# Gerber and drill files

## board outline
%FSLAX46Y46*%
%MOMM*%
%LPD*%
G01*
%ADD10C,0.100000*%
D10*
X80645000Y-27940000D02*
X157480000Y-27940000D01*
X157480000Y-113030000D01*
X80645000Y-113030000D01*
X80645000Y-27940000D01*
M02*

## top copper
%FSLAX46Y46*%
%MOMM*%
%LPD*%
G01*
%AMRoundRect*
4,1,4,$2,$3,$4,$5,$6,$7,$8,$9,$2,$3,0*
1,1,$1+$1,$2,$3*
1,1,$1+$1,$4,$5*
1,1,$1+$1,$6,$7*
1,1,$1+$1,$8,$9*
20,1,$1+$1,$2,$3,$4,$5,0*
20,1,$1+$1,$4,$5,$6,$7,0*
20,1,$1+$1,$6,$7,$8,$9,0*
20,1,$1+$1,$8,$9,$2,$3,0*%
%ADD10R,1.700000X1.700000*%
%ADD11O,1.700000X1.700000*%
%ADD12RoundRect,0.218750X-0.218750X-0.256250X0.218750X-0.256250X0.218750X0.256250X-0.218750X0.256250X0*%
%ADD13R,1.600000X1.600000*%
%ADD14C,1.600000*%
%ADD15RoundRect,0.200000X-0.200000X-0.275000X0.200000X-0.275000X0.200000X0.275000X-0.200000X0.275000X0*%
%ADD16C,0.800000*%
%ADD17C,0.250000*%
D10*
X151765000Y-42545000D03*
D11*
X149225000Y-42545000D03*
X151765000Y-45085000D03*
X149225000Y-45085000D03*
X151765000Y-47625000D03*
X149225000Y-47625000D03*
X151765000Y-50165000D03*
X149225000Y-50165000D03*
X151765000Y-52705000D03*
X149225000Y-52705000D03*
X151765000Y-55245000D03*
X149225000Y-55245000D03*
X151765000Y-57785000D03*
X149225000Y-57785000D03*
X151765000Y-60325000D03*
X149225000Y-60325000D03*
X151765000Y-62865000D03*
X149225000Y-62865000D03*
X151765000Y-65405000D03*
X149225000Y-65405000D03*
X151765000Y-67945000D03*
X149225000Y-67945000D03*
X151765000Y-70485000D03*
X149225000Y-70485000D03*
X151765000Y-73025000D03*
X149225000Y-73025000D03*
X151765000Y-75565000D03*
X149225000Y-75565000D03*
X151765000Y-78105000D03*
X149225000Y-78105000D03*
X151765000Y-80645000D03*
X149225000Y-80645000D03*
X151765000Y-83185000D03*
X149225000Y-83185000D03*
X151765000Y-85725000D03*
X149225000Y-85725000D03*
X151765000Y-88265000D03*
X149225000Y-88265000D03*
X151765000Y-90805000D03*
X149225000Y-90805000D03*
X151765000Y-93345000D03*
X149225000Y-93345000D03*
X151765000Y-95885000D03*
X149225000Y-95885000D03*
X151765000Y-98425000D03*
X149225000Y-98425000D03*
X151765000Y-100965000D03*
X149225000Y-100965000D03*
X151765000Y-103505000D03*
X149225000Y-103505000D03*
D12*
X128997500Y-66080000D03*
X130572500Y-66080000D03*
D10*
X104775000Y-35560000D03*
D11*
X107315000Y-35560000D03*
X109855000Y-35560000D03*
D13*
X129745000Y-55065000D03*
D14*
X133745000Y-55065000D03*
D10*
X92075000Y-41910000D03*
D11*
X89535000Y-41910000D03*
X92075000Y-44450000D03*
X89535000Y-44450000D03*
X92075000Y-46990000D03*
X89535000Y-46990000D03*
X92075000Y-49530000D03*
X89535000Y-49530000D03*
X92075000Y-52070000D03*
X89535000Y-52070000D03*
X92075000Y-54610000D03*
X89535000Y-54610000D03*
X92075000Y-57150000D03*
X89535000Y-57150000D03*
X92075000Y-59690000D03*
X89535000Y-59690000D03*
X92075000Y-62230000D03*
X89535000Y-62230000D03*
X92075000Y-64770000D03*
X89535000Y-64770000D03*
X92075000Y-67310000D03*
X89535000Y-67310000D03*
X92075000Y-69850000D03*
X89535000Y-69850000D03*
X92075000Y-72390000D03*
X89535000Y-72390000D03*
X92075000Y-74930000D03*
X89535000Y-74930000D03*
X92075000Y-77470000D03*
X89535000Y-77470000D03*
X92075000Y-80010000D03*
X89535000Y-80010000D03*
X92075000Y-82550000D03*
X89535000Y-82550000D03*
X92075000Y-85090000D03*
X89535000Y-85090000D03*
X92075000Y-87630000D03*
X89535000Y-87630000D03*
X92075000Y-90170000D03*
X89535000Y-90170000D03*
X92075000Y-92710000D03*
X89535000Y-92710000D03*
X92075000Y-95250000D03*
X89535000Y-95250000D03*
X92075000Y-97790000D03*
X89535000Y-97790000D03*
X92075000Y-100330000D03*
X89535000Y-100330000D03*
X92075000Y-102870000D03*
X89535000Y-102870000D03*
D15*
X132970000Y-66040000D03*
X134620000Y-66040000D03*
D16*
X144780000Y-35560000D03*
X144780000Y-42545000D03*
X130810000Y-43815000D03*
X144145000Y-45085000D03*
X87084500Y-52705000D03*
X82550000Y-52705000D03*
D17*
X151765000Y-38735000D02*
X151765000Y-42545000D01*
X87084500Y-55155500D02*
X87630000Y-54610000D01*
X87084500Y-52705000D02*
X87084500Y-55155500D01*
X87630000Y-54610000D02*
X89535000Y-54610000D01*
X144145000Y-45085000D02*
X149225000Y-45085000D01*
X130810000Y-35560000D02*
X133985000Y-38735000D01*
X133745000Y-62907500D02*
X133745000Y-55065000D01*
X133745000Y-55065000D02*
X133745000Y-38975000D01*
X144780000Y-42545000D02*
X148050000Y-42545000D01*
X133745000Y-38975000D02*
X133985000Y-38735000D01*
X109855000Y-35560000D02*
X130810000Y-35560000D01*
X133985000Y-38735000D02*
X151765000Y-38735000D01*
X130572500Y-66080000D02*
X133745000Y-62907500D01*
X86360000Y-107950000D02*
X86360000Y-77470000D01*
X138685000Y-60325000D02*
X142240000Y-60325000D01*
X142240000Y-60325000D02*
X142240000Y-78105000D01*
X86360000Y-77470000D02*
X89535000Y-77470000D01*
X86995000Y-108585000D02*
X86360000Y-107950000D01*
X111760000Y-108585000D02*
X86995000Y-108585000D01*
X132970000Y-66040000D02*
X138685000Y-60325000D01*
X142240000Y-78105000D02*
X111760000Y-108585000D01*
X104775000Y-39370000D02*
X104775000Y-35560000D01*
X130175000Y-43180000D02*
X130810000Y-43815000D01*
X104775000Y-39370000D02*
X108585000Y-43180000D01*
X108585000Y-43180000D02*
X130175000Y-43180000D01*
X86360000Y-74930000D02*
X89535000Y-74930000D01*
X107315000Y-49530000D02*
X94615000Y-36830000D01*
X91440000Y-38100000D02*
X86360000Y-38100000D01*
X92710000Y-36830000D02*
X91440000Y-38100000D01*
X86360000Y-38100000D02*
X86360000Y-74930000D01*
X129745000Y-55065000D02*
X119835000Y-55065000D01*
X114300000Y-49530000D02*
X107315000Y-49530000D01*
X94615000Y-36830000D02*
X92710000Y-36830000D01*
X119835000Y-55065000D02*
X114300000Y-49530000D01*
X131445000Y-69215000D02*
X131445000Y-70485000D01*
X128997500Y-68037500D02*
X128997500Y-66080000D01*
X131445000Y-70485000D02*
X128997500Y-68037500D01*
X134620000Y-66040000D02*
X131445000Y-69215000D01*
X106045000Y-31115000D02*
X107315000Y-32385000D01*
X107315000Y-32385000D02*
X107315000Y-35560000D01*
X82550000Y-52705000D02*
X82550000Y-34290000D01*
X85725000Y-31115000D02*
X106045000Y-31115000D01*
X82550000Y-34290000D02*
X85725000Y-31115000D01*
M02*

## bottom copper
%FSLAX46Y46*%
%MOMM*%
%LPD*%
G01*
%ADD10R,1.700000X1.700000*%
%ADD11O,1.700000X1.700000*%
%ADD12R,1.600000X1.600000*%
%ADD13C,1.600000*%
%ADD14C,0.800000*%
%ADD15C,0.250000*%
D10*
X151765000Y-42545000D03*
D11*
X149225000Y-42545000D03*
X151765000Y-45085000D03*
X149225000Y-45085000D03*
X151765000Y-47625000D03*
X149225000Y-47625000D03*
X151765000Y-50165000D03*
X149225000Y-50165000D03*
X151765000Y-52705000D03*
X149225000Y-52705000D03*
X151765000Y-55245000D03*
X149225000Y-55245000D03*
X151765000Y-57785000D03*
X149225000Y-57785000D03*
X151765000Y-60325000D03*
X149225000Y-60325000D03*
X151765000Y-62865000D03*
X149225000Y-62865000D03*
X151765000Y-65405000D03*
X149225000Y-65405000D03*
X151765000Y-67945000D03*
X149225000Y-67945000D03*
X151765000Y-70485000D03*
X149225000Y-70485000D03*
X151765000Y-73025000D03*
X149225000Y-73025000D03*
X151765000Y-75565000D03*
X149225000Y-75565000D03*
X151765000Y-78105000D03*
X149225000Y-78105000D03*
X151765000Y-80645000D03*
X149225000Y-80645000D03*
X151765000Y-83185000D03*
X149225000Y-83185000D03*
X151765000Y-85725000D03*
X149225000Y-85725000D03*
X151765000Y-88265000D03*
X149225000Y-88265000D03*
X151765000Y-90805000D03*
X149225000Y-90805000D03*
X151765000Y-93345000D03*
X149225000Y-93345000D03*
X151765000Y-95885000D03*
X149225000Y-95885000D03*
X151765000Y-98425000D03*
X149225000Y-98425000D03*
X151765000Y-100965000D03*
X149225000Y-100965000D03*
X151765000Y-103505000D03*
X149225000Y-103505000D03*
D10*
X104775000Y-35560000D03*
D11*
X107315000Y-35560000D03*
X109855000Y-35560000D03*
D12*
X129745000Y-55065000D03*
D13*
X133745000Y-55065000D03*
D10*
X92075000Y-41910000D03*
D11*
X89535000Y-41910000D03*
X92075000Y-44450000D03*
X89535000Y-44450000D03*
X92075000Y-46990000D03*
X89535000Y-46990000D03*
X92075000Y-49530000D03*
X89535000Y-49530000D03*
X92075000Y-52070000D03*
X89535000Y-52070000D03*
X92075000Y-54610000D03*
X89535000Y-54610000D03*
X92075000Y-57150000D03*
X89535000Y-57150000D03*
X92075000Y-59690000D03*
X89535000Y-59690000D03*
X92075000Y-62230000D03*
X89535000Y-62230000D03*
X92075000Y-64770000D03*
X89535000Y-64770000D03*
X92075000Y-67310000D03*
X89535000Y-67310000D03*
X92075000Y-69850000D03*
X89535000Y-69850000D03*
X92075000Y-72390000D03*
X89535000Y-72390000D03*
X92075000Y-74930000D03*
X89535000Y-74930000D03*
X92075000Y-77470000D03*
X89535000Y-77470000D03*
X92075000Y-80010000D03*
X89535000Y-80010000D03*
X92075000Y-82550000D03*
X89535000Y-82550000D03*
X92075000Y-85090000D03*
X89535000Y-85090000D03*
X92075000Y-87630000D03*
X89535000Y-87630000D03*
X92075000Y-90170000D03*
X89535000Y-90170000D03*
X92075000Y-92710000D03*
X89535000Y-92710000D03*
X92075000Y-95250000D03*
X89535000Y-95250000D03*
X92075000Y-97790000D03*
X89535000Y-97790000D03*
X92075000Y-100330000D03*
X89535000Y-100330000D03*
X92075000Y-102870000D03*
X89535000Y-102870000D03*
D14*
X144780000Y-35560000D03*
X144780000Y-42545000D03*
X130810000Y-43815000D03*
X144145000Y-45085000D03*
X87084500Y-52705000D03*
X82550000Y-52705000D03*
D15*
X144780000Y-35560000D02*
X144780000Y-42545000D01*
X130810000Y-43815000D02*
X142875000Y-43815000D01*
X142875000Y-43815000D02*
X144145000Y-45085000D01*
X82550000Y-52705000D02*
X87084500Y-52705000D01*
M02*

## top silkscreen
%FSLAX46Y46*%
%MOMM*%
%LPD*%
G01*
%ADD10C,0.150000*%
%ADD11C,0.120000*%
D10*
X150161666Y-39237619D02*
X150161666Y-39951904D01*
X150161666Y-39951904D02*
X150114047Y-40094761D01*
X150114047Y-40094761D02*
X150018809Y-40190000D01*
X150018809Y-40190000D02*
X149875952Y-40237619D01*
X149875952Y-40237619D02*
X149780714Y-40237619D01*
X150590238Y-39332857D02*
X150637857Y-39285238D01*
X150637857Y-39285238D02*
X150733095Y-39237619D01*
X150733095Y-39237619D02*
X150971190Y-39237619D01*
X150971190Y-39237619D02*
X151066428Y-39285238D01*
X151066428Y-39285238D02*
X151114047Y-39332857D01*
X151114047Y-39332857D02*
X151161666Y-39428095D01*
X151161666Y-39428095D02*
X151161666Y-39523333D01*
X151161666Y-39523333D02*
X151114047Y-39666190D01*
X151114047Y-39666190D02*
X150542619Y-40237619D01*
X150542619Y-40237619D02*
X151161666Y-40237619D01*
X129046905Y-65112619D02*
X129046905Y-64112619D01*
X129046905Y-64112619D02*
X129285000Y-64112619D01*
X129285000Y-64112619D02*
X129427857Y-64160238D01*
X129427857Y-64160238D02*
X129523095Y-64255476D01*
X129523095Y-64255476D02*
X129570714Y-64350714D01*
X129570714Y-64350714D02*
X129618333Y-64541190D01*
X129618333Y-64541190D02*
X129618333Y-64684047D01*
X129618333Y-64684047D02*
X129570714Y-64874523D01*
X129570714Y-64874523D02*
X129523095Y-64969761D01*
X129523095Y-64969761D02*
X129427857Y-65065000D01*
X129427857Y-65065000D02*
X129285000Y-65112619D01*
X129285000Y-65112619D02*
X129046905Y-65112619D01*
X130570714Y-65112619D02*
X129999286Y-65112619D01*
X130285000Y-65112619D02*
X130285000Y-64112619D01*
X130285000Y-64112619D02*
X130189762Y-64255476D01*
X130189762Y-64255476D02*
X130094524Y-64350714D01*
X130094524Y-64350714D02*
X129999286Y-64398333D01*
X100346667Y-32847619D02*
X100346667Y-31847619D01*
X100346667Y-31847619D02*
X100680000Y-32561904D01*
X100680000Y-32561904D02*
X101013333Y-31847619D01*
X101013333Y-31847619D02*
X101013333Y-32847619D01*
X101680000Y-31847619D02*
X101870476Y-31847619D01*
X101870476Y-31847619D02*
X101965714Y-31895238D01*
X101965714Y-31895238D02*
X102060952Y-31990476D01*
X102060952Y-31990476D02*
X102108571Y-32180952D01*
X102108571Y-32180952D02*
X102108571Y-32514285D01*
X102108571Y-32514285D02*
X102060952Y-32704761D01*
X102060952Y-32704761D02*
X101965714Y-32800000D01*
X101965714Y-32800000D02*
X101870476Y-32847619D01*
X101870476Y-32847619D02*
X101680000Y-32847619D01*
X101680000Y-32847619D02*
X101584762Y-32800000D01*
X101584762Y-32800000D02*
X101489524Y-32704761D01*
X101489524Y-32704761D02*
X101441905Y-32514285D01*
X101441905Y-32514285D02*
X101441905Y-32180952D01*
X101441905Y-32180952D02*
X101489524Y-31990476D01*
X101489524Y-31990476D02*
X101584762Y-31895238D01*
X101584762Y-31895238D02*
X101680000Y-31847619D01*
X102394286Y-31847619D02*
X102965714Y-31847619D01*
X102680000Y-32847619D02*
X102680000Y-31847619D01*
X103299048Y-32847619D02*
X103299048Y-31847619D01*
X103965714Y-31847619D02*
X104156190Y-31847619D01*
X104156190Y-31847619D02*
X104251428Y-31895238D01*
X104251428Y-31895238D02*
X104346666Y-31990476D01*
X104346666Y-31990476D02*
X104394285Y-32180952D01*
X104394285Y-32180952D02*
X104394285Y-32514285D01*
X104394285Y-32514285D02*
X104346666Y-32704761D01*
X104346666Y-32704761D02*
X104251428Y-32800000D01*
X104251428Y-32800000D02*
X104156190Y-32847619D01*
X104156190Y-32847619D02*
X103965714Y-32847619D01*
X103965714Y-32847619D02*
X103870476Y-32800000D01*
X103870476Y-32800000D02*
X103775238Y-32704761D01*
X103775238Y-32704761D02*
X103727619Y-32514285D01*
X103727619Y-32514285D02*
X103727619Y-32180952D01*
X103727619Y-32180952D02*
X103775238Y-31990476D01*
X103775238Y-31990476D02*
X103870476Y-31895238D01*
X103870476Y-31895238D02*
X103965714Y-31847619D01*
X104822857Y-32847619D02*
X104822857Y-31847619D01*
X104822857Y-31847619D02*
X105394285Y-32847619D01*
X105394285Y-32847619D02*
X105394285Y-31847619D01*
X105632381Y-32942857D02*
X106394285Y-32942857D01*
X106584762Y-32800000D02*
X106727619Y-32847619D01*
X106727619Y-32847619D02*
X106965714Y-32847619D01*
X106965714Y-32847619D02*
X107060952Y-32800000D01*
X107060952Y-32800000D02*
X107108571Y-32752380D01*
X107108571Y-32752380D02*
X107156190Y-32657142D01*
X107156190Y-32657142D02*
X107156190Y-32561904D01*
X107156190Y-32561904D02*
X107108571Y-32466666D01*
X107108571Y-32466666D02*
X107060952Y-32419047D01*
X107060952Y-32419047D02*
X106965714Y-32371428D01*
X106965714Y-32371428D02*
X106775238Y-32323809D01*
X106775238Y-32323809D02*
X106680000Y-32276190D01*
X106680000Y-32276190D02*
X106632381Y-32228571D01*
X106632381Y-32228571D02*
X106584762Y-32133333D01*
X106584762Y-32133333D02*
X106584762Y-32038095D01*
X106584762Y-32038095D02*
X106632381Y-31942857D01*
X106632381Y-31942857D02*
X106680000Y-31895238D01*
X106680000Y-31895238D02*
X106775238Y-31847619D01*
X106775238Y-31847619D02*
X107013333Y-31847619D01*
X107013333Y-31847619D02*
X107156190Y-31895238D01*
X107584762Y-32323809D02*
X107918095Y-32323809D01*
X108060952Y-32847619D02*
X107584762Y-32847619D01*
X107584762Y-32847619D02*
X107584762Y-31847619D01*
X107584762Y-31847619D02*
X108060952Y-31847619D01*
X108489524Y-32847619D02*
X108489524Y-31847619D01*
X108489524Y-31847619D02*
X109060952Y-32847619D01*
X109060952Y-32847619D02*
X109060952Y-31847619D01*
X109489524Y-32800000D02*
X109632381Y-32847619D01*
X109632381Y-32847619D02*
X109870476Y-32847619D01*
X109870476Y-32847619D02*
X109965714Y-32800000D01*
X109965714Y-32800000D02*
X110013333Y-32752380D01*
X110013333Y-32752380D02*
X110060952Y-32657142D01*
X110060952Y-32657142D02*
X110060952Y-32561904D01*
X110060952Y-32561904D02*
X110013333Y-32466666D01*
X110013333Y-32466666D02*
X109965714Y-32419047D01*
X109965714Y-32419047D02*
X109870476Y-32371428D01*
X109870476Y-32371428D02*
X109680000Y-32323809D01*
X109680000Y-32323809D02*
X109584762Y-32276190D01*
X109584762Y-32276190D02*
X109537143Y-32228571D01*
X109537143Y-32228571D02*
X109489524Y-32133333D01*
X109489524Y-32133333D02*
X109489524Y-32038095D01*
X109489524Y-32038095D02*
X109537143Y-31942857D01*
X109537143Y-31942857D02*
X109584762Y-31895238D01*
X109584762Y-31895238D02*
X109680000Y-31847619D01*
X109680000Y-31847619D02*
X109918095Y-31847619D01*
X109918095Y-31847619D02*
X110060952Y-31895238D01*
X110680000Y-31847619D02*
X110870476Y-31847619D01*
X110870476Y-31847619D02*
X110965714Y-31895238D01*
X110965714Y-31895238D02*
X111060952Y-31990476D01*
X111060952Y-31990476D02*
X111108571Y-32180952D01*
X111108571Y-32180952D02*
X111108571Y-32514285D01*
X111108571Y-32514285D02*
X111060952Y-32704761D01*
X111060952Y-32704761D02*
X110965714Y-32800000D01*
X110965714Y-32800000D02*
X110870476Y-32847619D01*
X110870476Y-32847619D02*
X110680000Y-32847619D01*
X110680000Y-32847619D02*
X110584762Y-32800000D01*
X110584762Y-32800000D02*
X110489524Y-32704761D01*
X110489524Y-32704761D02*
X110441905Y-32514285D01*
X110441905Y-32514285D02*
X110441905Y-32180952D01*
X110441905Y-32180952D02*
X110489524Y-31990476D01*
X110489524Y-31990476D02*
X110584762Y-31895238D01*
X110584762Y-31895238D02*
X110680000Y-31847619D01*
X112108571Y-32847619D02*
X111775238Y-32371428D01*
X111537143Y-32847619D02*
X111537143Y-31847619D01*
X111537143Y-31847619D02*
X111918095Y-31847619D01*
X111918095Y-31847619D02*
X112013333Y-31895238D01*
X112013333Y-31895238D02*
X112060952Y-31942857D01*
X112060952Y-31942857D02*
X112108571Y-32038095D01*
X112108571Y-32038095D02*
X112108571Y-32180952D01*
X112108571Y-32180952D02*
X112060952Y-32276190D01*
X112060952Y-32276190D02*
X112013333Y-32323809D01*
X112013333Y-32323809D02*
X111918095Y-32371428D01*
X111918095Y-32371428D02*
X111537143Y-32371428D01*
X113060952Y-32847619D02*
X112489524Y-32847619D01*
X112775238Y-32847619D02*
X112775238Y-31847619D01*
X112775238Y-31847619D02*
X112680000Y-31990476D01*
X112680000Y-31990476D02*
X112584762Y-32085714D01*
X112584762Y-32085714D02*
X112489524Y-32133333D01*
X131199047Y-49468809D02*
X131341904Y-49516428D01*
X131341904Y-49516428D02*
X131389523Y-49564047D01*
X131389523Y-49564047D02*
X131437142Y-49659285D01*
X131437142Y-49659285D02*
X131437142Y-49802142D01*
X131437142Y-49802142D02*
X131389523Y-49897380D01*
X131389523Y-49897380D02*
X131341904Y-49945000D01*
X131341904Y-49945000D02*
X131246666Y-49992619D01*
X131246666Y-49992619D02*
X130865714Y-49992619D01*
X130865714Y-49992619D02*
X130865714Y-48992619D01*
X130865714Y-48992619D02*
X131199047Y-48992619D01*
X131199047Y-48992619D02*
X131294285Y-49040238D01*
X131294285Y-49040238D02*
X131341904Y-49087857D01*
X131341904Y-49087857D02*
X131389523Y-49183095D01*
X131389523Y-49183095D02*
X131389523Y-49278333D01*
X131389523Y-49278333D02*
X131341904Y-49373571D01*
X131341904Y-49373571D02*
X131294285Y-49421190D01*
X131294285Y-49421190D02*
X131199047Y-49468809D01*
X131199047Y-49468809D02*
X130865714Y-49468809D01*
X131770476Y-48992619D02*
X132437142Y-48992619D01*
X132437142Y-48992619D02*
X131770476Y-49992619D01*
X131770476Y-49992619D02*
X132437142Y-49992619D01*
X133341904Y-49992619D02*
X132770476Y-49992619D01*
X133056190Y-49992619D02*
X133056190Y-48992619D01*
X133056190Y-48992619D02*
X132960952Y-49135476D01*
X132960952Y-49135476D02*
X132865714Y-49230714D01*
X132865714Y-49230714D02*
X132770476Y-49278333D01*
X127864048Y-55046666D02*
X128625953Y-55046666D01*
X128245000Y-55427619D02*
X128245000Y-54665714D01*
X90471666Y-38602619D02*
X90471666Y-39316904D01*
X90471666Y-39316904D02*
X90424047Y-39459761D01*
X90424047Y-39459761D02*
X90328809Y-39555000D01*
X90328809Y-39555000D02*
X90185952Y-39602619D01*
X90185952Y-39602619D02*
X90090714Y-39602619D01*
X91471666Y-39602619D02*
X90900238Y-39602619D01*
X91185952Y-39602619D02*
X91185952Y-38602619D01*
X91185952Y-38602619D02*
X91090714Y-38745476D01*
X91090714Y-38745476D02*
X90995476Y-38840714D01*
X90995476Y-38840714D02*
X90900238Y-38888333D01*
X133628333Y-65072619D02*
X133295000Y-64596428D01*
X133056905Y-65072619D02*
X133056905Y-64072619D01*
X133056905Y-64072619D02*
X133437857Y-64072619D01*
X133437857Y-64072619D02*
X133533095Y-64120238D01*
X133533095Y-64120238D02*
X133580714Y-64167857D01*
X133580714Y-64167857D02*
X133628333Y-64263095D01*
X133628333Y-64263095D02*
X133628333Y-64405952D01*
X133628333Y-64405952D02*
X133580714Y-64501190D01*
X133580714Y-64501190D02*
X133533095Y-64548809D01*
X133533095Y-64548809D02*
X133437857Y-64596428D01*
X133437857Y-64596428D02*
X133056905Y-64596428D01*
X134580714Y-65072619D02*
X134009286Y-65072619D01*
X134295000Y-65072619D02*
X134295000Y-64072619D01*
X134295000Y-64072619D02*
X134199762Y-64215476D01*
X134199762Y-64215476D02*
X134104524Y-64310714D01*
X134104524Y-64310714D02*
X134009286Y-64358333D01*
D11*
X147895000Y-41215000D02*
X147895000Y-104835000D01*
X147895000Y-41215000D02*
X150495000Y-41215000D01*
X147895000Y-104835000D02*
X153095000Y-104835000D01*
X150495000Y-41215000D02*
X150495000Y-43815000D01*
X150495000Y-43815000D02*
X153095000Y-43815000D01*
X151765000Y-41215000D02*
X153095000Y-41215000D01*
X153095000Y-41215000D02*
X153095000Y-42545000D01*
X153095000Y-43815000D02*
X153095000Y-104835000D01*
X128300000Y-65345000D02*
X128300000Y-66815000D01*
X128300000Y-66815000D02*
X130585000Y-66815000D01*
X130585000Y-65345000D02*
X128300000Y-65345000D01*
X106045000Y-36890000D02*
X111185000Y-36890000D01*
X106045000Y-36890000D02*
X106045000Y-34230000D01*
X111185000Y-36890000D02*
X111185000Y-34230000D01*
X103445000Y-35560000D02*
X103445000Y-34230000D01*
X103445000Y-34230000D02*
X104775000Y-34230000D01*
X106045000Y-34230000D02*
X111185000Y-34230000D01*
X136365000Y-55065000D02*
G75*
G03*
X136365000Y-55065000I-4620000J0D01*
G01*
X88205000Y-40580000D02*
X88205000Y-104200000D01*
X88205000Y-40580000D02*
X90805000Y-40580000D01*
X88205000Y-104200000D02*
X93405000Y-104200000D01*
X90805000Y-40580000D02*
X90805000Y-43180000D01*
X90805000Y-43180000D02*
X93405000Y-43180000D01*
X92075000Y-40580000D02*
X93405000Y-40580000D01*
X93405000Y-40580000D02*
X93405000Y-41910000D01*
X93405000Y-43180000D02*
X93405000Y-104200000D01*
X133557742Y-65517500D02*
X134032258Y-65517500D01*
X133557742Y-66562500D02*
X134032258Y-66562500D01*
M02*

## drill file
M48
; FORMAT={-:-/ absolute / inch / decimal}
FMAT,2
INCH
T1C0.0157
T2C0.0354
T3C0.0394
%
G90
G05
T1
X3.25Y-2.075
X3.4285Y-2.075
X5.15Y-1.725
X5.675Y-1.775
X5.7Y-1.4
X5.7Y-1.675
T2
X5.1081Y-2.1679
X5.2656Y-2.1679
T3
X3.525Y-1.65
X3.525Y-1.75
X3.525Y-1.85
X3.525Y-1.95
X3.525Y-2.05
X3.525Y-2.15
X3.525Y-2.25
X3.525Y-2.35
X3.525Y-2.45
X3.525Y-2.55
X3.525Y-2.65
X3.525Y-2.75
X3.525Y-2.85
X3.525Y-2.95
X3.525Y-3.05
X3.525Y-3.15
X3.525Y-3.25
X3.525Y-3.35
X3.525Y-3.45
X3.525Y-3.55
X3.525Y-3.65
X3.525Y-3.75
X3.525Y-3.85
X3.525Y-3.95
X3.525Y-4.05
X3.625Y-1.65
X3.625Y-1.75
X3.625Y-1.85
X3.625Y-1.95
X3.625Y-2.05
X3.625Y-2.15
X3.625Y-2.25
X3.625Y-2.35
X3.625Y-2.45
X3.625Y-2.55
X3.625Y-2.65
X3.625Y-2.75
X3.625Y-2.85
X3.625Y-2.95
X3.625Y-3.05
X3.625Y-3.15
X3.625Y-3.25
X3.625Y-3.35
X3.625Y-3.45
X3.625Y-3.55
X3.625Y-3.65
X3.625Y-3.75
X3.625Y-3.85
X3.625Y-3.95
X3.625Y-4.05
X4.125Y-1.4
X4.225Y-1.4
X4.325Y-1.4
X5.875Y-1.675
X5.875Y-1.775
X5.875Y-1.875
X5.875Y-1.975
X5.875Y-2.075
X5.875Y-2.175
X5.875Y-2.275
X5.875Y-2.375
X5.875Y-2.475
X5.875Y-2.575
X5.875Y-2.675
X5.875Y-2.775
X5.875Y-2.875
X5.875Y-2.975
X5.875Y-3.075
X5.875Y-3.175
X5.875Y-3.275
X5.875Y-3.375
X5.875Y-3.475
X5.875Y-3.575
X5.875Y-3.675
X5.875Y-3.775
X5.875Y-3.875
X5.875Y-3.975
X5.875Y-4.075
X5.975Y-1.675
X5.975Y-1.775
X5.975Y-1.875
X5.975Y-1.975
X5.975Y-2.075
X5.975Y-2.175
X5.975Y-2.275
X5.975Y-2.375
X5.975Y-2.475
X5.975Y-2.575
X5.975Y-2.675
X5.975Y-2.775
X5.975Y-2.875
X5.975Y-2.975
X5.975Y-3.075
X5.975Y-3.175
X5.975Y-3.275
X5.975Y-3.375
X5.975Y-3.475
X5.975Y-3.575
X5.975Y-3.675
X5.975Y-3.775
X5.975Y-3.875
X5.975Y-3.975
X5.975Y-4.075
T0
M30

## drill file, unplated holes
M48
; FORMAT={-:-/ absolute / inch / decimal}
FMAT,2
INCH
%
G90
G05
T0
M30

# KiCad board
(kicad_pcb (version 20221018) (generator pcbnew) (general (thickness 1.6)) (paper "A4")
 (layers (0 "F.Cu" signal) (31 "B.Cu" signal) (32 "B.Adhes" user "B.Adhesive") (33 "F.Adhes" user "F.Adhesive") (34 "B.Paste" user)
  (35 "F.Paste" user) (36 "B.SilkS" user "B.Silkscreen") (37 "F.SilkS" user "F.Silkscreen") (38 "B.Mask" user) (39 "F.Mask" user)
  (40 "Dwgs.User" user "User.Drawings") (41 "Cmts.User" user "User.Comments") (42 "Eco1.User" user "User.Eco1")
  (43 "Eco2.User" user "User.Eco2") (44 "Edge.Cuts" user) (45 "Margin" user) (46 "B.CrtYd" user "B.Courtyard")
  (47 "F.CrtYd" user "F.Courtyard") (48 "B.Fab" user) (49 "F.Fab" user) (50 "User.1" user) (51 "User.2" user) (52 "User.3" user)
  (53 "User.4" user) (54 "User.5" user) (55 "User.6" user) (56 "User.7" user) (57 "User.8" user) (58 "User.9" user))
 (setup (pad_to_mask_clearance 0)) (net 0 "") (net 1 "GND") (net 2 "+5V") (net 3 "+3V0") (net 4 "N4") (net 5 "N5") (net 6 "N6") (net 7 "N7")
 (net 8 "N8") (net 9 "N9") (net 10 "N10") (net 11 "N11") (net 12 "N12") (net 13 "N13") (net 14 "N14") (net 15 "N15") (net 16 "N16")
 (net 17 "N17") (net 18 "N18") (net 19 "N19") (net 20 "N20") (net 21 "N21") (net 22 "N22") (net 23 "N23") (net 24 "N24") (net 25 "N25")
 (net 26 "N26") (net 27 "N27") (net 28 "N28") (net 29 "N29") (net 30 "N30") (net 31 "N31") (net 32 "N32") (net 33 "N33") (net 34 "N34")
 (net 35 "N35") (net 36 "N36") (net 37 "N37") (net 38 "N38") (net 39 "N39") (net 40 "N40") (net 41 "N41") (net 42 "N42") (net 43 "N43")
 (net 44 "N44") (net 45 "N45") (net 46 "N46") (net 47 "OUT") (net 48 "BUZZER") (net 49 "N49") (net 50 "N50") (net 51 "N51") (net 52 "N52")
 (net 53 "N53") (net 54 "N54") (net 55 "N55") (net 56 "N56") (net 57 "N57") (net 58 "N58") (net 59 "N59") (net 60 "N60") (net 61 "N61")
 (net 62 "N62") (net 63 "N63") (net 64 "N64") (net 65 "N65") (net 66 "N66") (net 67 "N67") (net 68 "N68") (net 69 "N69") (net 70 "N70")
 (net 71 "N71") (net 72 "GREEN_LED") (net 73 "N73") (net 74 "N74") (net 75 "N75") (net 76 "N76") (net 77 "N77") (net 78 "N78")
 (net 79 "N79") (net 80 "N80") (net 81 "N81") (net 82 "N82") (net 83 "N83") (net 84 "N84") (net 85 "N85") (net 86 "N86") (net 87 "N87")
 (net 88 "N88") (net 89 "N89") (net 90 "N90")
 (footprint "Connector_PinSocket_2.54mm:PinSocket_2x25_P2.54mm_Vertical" (layer "F.Cu") (at 151.765 42.545)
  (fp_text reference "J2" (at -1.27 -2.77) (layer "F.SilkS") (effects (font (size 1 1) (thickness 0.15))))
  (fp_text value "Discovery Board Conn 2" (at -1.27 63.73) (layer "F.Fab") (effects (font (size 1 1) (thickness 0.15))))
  (fp_line (start -3.87 -1.33) (end -3.87 62.29) (stroke (width 0.12) (type solid)) (layer "F.SilkS"))
  (fp_line (start -3.87 -1.33) (end -1.27 -1.33) (stroke (width 0.12) (type solid)) (layer "F.SilkS"))
  (fp_line (start -3.87 62.29) (end 1.33 62.29) (stroke (width 0.12) (type solid)) (layer "F.SilkS"))
  (fp_line (start -1.27 -1.33) (end -1.27 1.27) (stroke (width 0.12) (type solid)) (layer "F.SilkS"))
  (fp_line (start -1.27 1.27) (end 1.33 1.27) (stroke (width 0.12) (type solid)) (layer "F.SilkS"))
  (fp_line (start 0 -1.33) (end 1.33 -1.33) (stroke (width 0.12) (type solid)) (layer "F.SilkS"))
  (fp_line (start 1.33 -1.33) (end 1.33 0) (stroke (width 0.12) (type solid)) (layer "F.SilkS"))
  (fp_line (start 1.33 1.27) (end 1.33 62.29) (stroke (width 0.12) (type solid)) (layer "F.SilkS"))
  (pad "1" thru_hole rect (at 0 0) (size 1.7 1.7) (drill 1) (layers "*.Cu" "*.Mask") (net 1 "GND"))
  (pad "2" thru_hole oval (at -2.54 0) (size 1.7 1.7) (drill 1) (layers "*.Cu" "*.Mask") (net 1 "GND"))
  (pad "3" thru_hole oval (at 0 2.54) (size 1.7 1.7) (drill 1) (layers "*.Cu" "*.Mask") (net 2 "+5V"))
  (pad "4" thru_hole oval (at -2.54 2.54) (size 1.7 1.7) (drill 1) (layers "*.Cu" "*.Mask") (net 2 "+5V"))
  (pad "5" thru_hole oval (at 0 5.08) (size 1.7 1.7) (drill 1) (layers "*.Cu" "*.Mask") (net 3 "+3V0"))
  (pad "6" thru_hole oval (at -2.54 5.08) (size 1.7 1.7) (drill 1) (layers "*.Cu" "*.Mask") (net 3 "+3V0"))
  (pad "7" thru_hole oval (at 0 7.62) (size 1.7 1.7) (drill 1) (layers "*.Cu" "*.Mask") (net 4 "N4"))
  (pad "8" thru_hole oval (at -2.54 7.62) (size 1.7 1.7) (drill 1) (layers "*.Cu" "*.Mask") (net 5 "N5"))
  (pad "9" thru_hole oval (at 0 10.16) (size 1.7 1.7) (drill 1) (layers "*.Cu" "*.Mask") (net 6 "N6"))
  (pad "10" thru_hole oval (at -2.54 10.16) (size 1.7 1.7) (drill 1) (layers "*.Cu" "*.Mask") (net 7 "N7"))
  (pad "11" thru_hole oval (at 0 12.7) (size 1.7 1.7) (drill 1) (layers "*.Cu" "*.Mask") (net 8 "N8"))
  (pad "12" thru_hole oval (at -2.54 12.7) (size 1.7 1.7) (drill 1) (layers "*.Cu" "*.Mask") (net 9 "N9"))
  (pad "13" thru_hole oval (at 0 15.24) (size 1.7 1.7) (drill 1) (layers "*.Cu" "*.Mask") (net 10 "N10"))
  (pad "14" thru_hole oval (at -2.54 15.24) (size 1.7 1.7) (drill 1) (layers "*.Cu" "*.Mask") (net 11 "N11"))
  (pad "15" thru_hole oval (at 0 17.78) (size 1.7 1.7) (drill 1) (layers "*.Cu" "*.Mask") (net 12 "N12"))
  (pad "16" thru_hole oval (at -2.54 17.78) (size 1.7 1.7) (drill 1) (layers "*.Cu" "*.Mask") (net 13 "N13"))
  (pad "17" thru_hole oval (at 0 20.32) (size 1.7 1.7) (drill 1) (layers "*.Cu" "*.Mask") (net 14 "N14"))
  (pad "18" thru_hole oval (at -2.54 20.32) (size 1.7 1.7) (drill 1) (layers "*.Cu" "*.Mask") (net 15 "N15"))
  (pad "19" thru_hole oval (at 0 22.86) (size 1.7 1.7) (drill 1) (layers "*.Cu" "*.Mask") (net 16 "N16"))
  (pad "20" thru_hole oval (at -2.54 22.86) (size 1.7 1.7) (drill 1) (layers "*.Cu" "*.Mask") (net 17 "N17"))
  (pad "21" thru_hole oval (at 0 25.4) (size 1.7 1.7) (drill 1) (layers "*.Cu" "*.Mask") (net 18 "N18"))
  (pad "22" thru_hole oval (at -2.54 25.4) (size 1.7 1.7) (drill 1) (layers "*.Cu" "*.Mask") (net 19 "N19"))
  (pad "23" thru_hole oval (at 0 27.94) (size 1.7 1.7) (drill 1) (layers "*.Cu" "*.Mask") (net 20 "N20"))
  (pad "24" thru_hole oval (at -2.54 27.94) (size 1.7 1.7) (drill 1) (layers "*.Cu" "*.Mask") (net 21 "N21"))
  (pad "25" thru_hole oval (at 0 30.48) (size 1.7 1.7) (drill 1) (layers "*.Cu" "*.Mask") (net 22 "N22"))
  (pad "26" thru_hole oval (at -2.54 30.48) (size 1.7 1.7) (drill 1) (layers "*.Cu" "*.Mask") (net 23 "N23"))
  (pad "27" thru_hole oval (at 0 33.02) (size 1.7 1.7) (drill 1) (layers "*.Cu" "*.Mask") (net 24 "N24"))
  (pad "28" thru_hole oval (at -2.54 33.02) (size 1.7 1.7) (drill 1) (layers "*.Cu" "*.Mask") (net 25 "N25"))
  (pad "29" thru_hole oval (at 0 35.56) (size 1.7 1.7) (drill 1) (layers "*.Cu" "*.Mask") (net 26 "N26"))
  (pad "30" thru_hole oval (at -2.54 35.56) (size 1.7 1.7) (drill 1) (layers "*.Cu" "*.Mask") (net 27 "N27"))
  (pad "31" thru_hole oval (at 0 38.1) (size 1.7 1.7) (drill 1) (layers "*.Cu" "*.Mask") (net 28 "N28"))
  (pad "32" thru_hole oval (at -2.54 38.1) (size 1.7 1.7) (drill 1) (layers "*.Cu" "*.Mask") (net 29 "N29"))
  (pad "33" thru_hole oval (at 0 40.64) (size 1.7 1.7) (drill 1) (layers "*.Cu" "*.Mask") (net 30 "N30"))
  (pad "34" thru_hole oval (at -2.54 40.64) (size 1.7 1.7) (drill 1) (layers "*.Cu" "*.Mask") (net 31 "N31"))
  (pad "35" thru_hole oval (at 0 43.18) (size 1.7 1.7) (drill 1) (layers "*.Cu" "*.Mask") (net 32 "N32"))
  (pad "36" thru_hole oval (at -2.54 43.18) (size 1.7 1.7) (drill 1) (layers "*.Cu" "*.Mask") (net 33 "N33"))
  (pad "37" thru_hole oval (at 0 45.72) (size 1.7 1.7) (drill 1) (layers "*.Cu" "*.Mask") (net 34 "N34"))
  (pad "38" thru_hole oval (at -2.54 45.72) (size 1.7 1.7) (drill 1) (layers "*.Cu" "*.Mask") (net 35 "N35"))
  (pad "39" thru_hole oval (at 0 48.26) (size 1.7 1.7) (drill 1) (layers "*.Cu" "*.Mask") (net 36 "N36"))
  (pad "40" thru_hole oval (at -2.54 48.26) (size 1.7 1.7) (drill 1) (layers "*.Cu" "*.Mask") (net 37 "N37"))
  (pad "41" thru_hole oval (at 0 50.8) (size 1.7 1.7) (drill 1) (layers "*.Cu" "*.Mask") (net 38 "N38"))
  (pad "42" thru_hole oval (at -2.54 50.8) (size 1.7 1.7) (drill 1) (layers "*.Cu" "*.Mask") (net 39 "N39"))
  (pad "43" thru_hole oval (at 0 53.34) (size 1.7 1.7) (drill 1) (layers "*.Cu" "*.Mask") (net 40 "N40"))
  (pad "44" thru_hole oval (at -2.54 53.34) (size 1.7 1.7) (drill 1) (layers "*.Cu" "*.Mask") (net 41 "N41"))
  (pad "45" thru_hole oval (at 0 55.88) (size 1.7 1.7) (drill 1) (layers "*.Cu" "*.Mask") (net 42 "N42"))
  (pad "46" thru_hole oval (at -2.54 55.88) (size 1.7 1.7) (drill 1) (layers "*.Cu" "*.Mask") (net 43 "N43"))
  (pad "47" thru_hole oval (at 0 58.42) (size 1.7 1.7) (drill 1) (layers "*.Cu" "*.Mask") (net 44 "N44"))
  (pad "48" thru_hole oval (at -2.54 58.42) (size 1.7 1.7) (drill 1) (layers "*.Cu" "*.Mask") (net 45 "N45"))
  (pad "49" thru_hole oval (at 0 60.96) (size 1.7 1.7) (drill 1) (layers "*.Cu" "*.Mask") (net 1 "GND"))
  (pad "50" thru_hole oval (at -2.54 60.96) (size 1.7 1.7) (drill 1) (layers "*.Cu" "*.Mask") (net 1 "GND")))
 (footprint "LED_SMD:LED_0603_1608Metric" (layer "F.Cu") (at 129.785 66.08)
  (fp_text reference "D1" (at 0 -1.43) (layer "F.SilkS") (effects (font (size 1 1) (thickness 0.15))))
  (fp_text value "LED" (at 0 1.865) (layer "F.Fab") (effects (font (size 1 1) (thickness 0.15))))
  (fp_line (start -1.485 -0.735) (end -1.485 0.735) (stroke (width 0.12) (type solid)) (layer "F.SilkS"))
  (fp_line (start -1.485 0.735) (end 0.8 0.735) (stroke (width 0.12) (type solid)) (layer "F.SilkS"))
  (fp_line (start 0.8 -0.735) (end -1.485 -0.735) (stroke (width 0.12) (type solid)) (layer "F.SilkS"))
  (pad "1" smd roundrect (at -0.7875 0) (size 0.875 0.95) (layers "F.Cu" "F.Paste" "F.Mask") (roundrect_rratio 0.25) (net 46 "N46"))
  (pad "2" smd roundrect (at 0.7875 0) (size 0.875 0.95) (layers "F.Cu" "F.Paste" "F.Mask") (roundrect_rratio 0.25) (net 1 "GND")))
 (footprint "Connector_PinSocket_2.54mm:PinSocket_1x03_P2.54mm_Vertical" (layer "F.Cu") (at 104.775 35.56 90)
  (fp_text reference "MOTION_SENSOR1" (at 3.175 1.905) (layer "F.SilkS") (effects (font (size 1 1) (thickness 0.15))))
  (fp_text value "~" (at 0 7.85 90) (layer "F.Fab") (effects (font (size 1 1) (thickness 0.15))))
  (fp_line (start -1.33 1.27) (end -1.33 6.41) (stroke (width 0.12) (type solid)) (layer "F.SilkS"))
  (fp_line (start -1.33 1.27) (end 1.33 1.27) (stroke (width 0.12) (type solid)) (layer "F.SilkS"))
  (fp_line (start -1.33 6.41) (end 1.33 6.41) (stroke (width 0.12) (type solid)) (layer "F.SilkS"))
  (fp_line (start 0 -1.33) (end 1.33 -1.33) (stroke (width 0.12) (type solid)) (layer "F.SilkS"))
  (fp_line (start 1.33 -1.33) (end 1.33 0) (stroke (width 0.12) (type solid)) (layer "F.SilkS"))
  (fp_line (start 1.33 1.27) (end 1.33 6.41) (stroke (width 0.12) (type solid)) (layer "F.SilkS"))
  (pad "1" thru_hole rect (at 0 0 90) (size 1.7 1.7) (drill 1) (layers "*.Cu" "*.Mask") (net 2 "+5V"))
  (pad "2" thru_hole oval (at 0 2.54 90) (size 1.7 1.7) (drill 1) (layers "*.Cu" "*.Mask") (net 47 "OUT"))
  (pad "3" thru_hole oval (at 0 5.08 90) (size 1.7 1.7) (drill 1) (layers "*.Cu" "*.Mask") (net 1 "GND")))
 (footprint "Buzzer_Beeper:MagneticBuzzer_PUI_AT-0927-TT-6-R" (layer "F.Cu") (at 129.745 55.065)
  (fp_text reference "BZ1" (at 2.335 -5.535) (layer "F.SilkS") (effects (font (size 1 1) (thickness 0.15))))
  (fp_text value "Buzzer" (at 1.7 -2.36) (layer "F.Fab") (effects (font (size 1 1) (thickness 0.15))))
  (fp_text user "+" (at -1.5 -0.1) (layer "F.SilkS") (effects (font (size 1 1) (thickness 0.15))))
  (fp_circle (center 2 0) (end 6.62 0) (stroke (width 0.12) (type solid)) (fill none) (layer "F.SilkS"))
  (pad "1" thru_hole rect (at 0 0) (size 1.6 1.6) (drill 0.9) (layers "*.Cu" "*.Mask") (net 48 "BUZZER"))
  (pad "2" thru_hole circle (at 4 0) (size 1.6 1.6) (drill 0.9) (layers "*.Cu" "*.Mask") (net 1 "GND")))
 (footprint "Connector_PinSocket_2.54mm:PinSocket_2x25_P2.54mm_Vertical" (layer "F.Cu") (at 92.075 41.91)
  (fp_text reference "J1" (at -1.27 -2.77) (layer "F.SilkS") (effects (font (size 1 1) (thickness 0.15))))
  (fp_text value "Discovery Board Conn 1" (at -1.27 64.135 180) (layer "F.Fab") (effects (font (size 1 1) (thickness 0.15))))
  (fp_line (start -3.87 -1.33) (end -3.87 62.29) (stroke (width 0.12) (type solid)) (layer "F.SilkS"))
  (fp_line (start -3.87 -1.33) (end -1.27 -1.33) (stroke (width 0.12) (type solid)) (layer "F.SilkS"))
  (fp_line (start -3.87 62.29) (end 1.33 62.29) (stroke (width 0.12) (type solid)) (layer "F.SilkS"))
  (fp_line (start -1.27 -1.33) (end -1.27 1.27) (stroke (width 0.12) (type solid)) (layer "F.SilkS"))
  (fp_line (start -1.27 1.27) (end 1.33 1.27) (stroke (width 0.12) (type solid)) (layer "F.SilkS"))
  (fp_line (start 0 -1.33) (end 1.33 -1.33) (stroke (width 0.12) (type solid)) (layer "F.SilkS"))
  (fp_line (start 1.33 -1.33) (end 1.33 0) (stroke (width 0.12) (type solid)) (layer "F.SilkS"))
  (fp_line (start 1.33 1.27) (end 1.33 62.29) (stroke (width 0.12) (type solid)) (layer "F.SilkS"))
  (pad "1" thru_hole rect (at 0 0) (size 1.7 1.7) (drill 1) (layers "*.Cu" "*.Mask") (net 1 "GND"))
  (pad "2" thru_hole oval (at -2.54 0) (size 1.7 1.7) (drill 1) (layers "*.Cu" "*.Mask") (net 1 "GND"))
  (pad "3" thru_hole oval (at 0 2.54) (size 1.7 1.7) (drill 1) (layers "*.Cu" "*.Mask") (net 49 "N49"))
  (pad "4" thru_hole oval (at -2.54 2.54) (size 1.7 1.7) (drill 1) (layers "*.Cu" "*.Mask") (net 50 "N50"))
  (pad "5" thru_hole oval (at 0 5.08) (size 1.7 1.7) (drill 1) (layers "*.Cu" "*.Mask") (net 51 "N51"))
  (pad "6" thru_hole oval (at -2.54 5.08) (size 1.7 1.7) (drill 1) (layers "*.Cu" "*.Mask") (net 1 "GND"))
  (pad "7" thru_hole oval (at 0 7.62) (size 1.7 1.7) (drill 1) (layers "*.Cu" "*.Mask") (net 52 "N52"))
  (pad "8" thru_hole oval (at -2.54 7.62) (size 1.7 1.7) (drill 1) (layers "*.Cu" "*.Mask") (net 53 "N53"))
  (pad "9" thru_hole oval (at 0 10.16) (size 1.7 1.7) (drill 1) (layers "*.Cu" "*.Mask") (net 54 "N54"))
  (pad "10" thru_hole oval (at -2.54 10.16) (size 1.7 1.7) (drill 1) (layers "*.Cu" "*.Mask") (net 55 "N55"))
  (pad "11" thru_hole oval (at 0 12.7) (size 1.7 1.7) (drill 1) (layers "*.Cu" "*.Mask") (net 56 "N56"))
  (pad "12" thru_hole oval (at -2.54 12.7) (size 1.7 1.7) (drill 1) (layers "*.Cu" "*.Mask") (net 47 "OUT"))
  (pad "13" thru_hole oval (at 0 15.24) (size 1.7 1.7) (drill 1) (layers "*.Cu" "*.Mask") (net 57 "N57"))
  (pad "14" thru_hole oval (at -2.54 15.24) (size 1.7 1.7) (drill 1) (layers "*.Cu" "*.Mask") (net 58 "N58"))
  (pad "15" thru_hole oval (at 0 17.78) (size 1.7 1.7) (drill 1) (layers "*.Cu" "*.Mask") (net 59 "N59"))
  (pad "16" thru_hole oval (at -2.54 17.78) (size 1.7 1.7) (drill 1) (layers "*.Cu" "*.Mask") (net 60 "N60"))
  (pad "17" thru_hole oval (at 0 20.32) (size 1.7 1.7) (drill 1) (layers "*.Cu" "*.Mask") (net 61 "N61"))
  (pad "18" thru_hole oval (at -2.54 20.32) (size 1.7 1.7) (drill 1) (layers "*.Cu" "*.Mask") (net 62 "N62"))
  (pad "19" thru_hole oval (at 0 22.86) (size 1.7 1.7) (drill 1) (layers "*.Cu" "*.Mask") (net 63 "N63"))
  (pad "20" thru_hole oval (at -2.54 22.86) (size 1.7 1.7) (drill 1) (layers "*.Cu" "*.Mask") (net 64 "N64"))
  (pad "21" thru_hole oval (at 0 25.4) (size 1.7 1.7) (drill 1) (layers "*.Cu" "*.Mask") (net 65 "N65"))
  (pad "22" thru_hole oval (at -2.54 25.4) (size 1.7 1.7) (drill 1) (layers "*.Cu" "*.Mask") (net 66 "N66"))
  (pad "23" thru_hole oval (at 0 27.94) (size 1.7 1.7) (drill 1) (layers "*.Cu" "*.Mask") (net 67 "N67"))
  (pad "24" thru_hole oval (at -2.54 27.94) (size 1.7 1.7) (drill 1) (layers "*.Cu" "*.Mask") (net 1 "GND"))
  (pad "25" thru_hole oval (at 0 30.48) (size 1.7 1.7) (drill 1) (layers "*.Cu" "*.Mask") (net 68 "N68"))
  (pad "26" thru_hole oval (at -2.54 30.48) (size 1.7 1.7) (drill 1) (layers "*.Cu" "*.Mask") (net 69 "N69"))
  (pad "27" thru_hole oval (at 0 33.02) (size 1.7 1.7) (drill 1) (layers "*.Cu" "*.Mask") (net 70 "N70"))
  (pad "28" thru_hole oval (at -2.54 33.02) (size 1.7 1.7) (drill 1) (layers "*.Cu" "*.Mask") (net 48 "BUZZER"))
  (pad "29" thru_hole oval (at 0 35.56) (size 1.7 1.7) (drill 1) (layers "*.Cu" "*.Mask") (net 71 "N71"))
  (pad "30" thru_hole oval (at -2.54 35.56) (size 1.7 1.7) (drill 1) (layers "*.Cu" "*.Mask") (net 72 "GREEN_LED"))
  (pad "31" thru_hole oval (at 0 38.1) (size 1.7 1.7) (drill 1) (layers "*.Cu" "*.Mask") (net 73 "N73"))
  (pad "32" thru_hole oval (at -2.54 38.1) (size 1.7 1.7) (drill 1) (layers "*.Cu" "*.Mask") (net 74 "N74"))
  (pad "33" thru_hole oval (at 0 40.64) (size 1.7 1.7) (drill 1) (layers "*.Cu" "*.Mask") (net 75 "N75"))
  (pad "34" thru_hole oval (at -2.54 40.64) (size 1.7 1.7) (drill 1) (layers "*.Cu" "*.Mask") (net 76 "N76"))
  (pad "35" thru_hole oval (at 0 43.18) (size 1.7 1.7) (drill 1) (layers "*.Cu" "*.Mask") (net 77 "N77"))
  (pad "36" thru_hole oval (at -2.54 43.18) (size 1.7 1.7) (drill 1) (layers "*.Cu" "*.Mask") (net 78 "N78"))
  (pad "37" thru_hole oval (at 0 45.72) (size 1.7 1.7) (drill 1) (layers "*.Cu" "*.Mask") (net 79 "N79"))
  (pad "38" thru_hole oval (at -2.54 45.72) (size 1.7 1.7) (drill 1) (layers "*.Cu" "*.Mask") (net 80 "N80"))
  (pad "39" thru_hole oval (at 0 48.26) (size 1.7 1.7) (drill 1) (layers "*.Cu" "*.Mask") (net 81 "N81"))
  (pad "40" thru_hole oval (at -2.54 48.26) (size 1.7 1.7) (drill 1) (layers "*.Cu" "*.Mask") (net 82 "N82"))
  (pad "41" thru_hole oval (at 0 50.8) (size 1.7 1.7) (drill 1) (layers "*.Cu" "*.Mask") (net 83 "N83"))
  (pad "42" thru_hole oval (at -2.54 50.8) (size 1.7 1.7) (drill 1) (layers "*.Cu" "*.Mask") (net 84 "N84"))
  (pad "43" thru_hole oval (at 0 53.34) (size 1.7 1.7) (drill 1) (layers "*.Cu" "*.Mask") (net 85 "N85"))
  (pad "44" thru_hole oval (at -2.54 53.34) (size 1.7 1.7) (drill 1) (layers "*.Cu" "*.Mask") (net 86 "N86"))
  (pad "45" thru_hole oval (at 0 55.88) (size 1.7 1.7) (drill 1) (layers "*.Cu" "*.Mask") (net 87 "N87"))
  (pad "46" thru_hole oval (at -2.54 55.88) (size 1.7 1.7) (drill 1) (layers "*.Cu" "*.Mask") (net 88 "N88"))
  (pad "47" thru_hole oval (at 0 58.42) (size 1.7 1.7) (drill 1) (layers "*.Cu" "*.Mask") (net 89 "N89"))
  (pad "48" thru_hole oval (at -2.54 58.42) (size 1.7 1.7) (drill 1) (layers "*.Cu" "*.Mask") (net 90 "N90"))
  (pad "49" thru_hole oval (at 0 60.96) (size 1.7 1.7) (drill 1) (layers "*.Cu" "*.Mask") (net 1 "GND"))
  (pad "50" thru_hole oval (at -2.54 60.96) (size 1.7 1.7) (drill 1) (layers "*.Cu" "*.Mask") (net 1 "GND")))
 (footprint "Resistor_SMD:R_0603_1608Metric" (layer "F.Cu") (at 133.795 66.04)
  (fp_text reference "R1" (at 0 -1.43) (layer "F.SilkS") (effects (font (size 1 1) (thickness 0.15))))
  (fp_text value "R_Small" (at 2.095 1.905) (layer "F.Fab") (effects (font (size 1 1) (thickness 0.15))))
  (fp_line (start -0.237258 -0.5225) (end 0.237258 -0.5225) (stroke (width 0.12) (type solid)) (layer "F.SilkS"))
  (fp_line (start -0.237258 0.5225) (end 0.237258 0.5225) (stroke (width 0.12) (type solid)) (layer "F.SilkS"))
  (pad "1" smd roundrect (at -0.825 0) (size 0.8 0.95) (layers "F.Cu" "F.Paste" "F.Mask") (roundrect_rratio 0.25) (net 72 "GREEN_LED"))
  (pad "2" smd roundrect (at 0.825 0) (size 0.8 0.95) (layers "F.Cu" "F.Paste" "F.Mask") (roundrect_rratio 0.25) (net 46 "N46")))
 (gr_rect (start 80.645 27.94) (end 157.48 113.03) (stroke (width 0.1) (type default)) (fill none) (layer "Edge.Cuts"))
 (segment (start 130.81 35.56) (end 133.985 38.735) (width 0.25) (layer "F.Cu") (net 1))
 (segment (start 133.745 62.9075) (end 133.745 55.065) (width 0.25) (layer "F.Cu") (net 1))
 (segment (start 133.745 55.065) (end 133.745 38.975) (width 0.25) (layer "F.Cu") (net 1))
 (segment (start 144.78 42.545) (end 148.05 42.545) (width 0.25) (layer "F.Cu") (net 1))
 (segment (start 133.745 38.975) (end 133.985 38.735) (width 0.25) (layer "F.Cu") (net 1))
 (segment (start 109.855 35.56) (end 130.81 35.56) (width 0.25) (layer "F.Cu") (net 1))
 (segment (start 151.765 38.735) (end 151.765 42.545) (width 0.25) (layer "F.Cu") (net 1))
 (segment (start 133.985 38.735) (end 151.765 38.735) (width 0.25) (layer "F.Cu") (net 1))
 (segment (start 130.5725 66.08) (end 133.745 62.9075) (width 0.25) (layer "F.Cu") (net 1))
 (via (at 144.78 35.56) (size 0.8) (drill 0.4) (layers "F.Cu" "B.Cu") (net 1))
 (via (at 144.78 42.545) (size 0.8) (drill 0.4) (layers "F.Cu" "B.Cu") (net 1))
 (segment (start 144.78 35.56) (end 144.78 42.545) (width 0.25) (layer "B.Cu") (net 1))
 (segment (start 86.36 107.95) (end 86.36 77.47) (width 0.25) (layer "F.Cu") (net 72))
 (segment (start 138.685 60.325) (end 142.24 60.325) (width 0.25) (layer "F.Cu") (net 72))
 (segment (start 142.24 60.325) (end 142.24 78.105) (width 0.25) (layer "F.Cu") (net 72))
 (segment (start 86.36 77.47) (end 89.535 77.47) (width 0.25) (layer "F.Cu") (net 72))
 (segment (start 86.995 108.585) (end 86.36 107.95) (width 0.25) (layer "F.Cu") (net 72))
 (segment (start 111.76 108.585) (end 86.995 108.585) (width 0.25) (layer "F.Cu") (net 72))
 (segment (start 132.97 66.04) (end 138.685 60.325) (width 0.25) (layer "F.Cu") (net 72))
 (segment (start 142.24 78.105) (end 111.76 108.585) (width 0.25) (layer "F.Cu") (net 72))
 (segment (start 144.145 45.085) (end 149.225 45.085) (width 0.25) (layer "F.Cu") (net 2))
 (segment (start 104.775 39.37) (end 104.775 35.56) (width 0.25) (layer "F.Cu") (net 2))
 (segment (start 130.175 43.18) (end 130.81 43.815) (width 0.25) (layer "F.Cu") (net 2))
 (segment (start 104.775 39.37) (end 108.585 43.18) (width 0.25) (layer "F.Cu") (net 2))
 (segment (start 108.585 43.18) (end 130.175 43.18) (width 0.25) (layer "F.Cu") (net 2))
 (via (at 130.81 43.815) (size 0.8) (drill 0.4) (layers "F.Cu" "B.Cu") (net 2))
 (via (at 144.145 45.085) (size 0.8) (drill 0.4) (layers "F.Cu" "B.Cu") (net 2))
 (segment (start 130.81 43.815) (end 142.875 43.815) (width 0.25) (layer "B.Cu") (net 2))
 (segment (start 142.875 43.815) (end 144.145 45.085) (width 0.25) (layer "B.Cu") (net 2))
 (segment (start 86.36 74.93) (end 89.535 74.93) (width 0.25) (layer "F.Cu") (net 48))
 (segment (start 107.315 49.53) (end 94.615 36.83) (width 0.25) (layer "F.Cu") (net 48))
 (segment (start 91.44 38.1) (end 86.36 38.1) (width 0.25) (layer "F.Cu") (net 48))
 (segment (start 92.71 36.83) (end 91.44 38.1) (width 0.25) (layer "F.Cu") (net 48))
 (segment (start 86.36 38.1) (end 86.36 74.93) (width 0.25) (layer "F.Cu") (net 48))
 (segment (start 129.745 55.065) (end 119.835 55.065) (width 0.25) (layer "F.Cu") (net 48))
 (segment (start 114.3 49.53) (end 107.315 49.53) (width 0.25) (layer "F.Cu") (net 48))
 (segment (start 94.615 36.83) (end 92.71 36.83) (width 0.25) (layer "F.Cu") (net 48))
 (segment (start 119.835 55.065) (end 114.3 49.53) (width 0.25) (layer "F.Cu") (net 48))
 (segment (start 131.445 69.215) (end 131.445 70.485) (width 0.25) (layer "F.Cu") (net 46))
 (segment (start 128.9975 68.0375) (end 128.9975 66.08) (width 0.25) (layer "F.Cu") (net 46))
 (segment (start 131.445 70.485) (end 128.9975 68.0375) (width 0.25) (layer "F.Cu") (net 46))
 (segment (start 134.62 66.04) (end 131.445 69.215) (width 0.25) (layer "F.Cu") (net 46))
 (segment (start 106.045 31.115) (end 107.315 32.385) (width 0.25) (layer "F.Cu") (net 47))
 (segment (start 87.63 54.61) (end 89.535 54.61) (width 0.25) (layer "F.Cu") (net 47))
 (segment (start 107.315 32.385) (end 107.315 35.56) (width 0.25) (layer "F.Cu") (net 47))
 (segment (start 82.55 52.705) (end 82.55 34.29) (width 0.25) (layer "F.Cu") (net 47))
 (segment (start 85.725 31.115) (end 106.045 31.115) (width 0.25) (layer "F.Cu") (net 47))
 (segment (start 82.55 34.29) (end 85.725 31.115) (width 0.25) (layer "F.Cu") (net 47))
 (segment (start 87.0845 52.705) (end 87.0845 55.1555) (width 0.25) (layer "F.Cu") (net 47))
 (segment (start 87.0845 55.1555) (end 87.63 54.61) (width 0.25) (layer "F.Cu") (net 47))
 (via (at 87.0845 52.705) (size 0.8) (drill 0.4) (layers "F.Cu" "B.Cu") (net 47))
 (via (at 82.55 52.705) (size 0.8) (drill 0.4) (layers "F.Cu" "B.Cu") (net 47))
 (segment (start 82.55 52.705) (end 87.0845 52.705) (width 0.25) (layer "B.Cu") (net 47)))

